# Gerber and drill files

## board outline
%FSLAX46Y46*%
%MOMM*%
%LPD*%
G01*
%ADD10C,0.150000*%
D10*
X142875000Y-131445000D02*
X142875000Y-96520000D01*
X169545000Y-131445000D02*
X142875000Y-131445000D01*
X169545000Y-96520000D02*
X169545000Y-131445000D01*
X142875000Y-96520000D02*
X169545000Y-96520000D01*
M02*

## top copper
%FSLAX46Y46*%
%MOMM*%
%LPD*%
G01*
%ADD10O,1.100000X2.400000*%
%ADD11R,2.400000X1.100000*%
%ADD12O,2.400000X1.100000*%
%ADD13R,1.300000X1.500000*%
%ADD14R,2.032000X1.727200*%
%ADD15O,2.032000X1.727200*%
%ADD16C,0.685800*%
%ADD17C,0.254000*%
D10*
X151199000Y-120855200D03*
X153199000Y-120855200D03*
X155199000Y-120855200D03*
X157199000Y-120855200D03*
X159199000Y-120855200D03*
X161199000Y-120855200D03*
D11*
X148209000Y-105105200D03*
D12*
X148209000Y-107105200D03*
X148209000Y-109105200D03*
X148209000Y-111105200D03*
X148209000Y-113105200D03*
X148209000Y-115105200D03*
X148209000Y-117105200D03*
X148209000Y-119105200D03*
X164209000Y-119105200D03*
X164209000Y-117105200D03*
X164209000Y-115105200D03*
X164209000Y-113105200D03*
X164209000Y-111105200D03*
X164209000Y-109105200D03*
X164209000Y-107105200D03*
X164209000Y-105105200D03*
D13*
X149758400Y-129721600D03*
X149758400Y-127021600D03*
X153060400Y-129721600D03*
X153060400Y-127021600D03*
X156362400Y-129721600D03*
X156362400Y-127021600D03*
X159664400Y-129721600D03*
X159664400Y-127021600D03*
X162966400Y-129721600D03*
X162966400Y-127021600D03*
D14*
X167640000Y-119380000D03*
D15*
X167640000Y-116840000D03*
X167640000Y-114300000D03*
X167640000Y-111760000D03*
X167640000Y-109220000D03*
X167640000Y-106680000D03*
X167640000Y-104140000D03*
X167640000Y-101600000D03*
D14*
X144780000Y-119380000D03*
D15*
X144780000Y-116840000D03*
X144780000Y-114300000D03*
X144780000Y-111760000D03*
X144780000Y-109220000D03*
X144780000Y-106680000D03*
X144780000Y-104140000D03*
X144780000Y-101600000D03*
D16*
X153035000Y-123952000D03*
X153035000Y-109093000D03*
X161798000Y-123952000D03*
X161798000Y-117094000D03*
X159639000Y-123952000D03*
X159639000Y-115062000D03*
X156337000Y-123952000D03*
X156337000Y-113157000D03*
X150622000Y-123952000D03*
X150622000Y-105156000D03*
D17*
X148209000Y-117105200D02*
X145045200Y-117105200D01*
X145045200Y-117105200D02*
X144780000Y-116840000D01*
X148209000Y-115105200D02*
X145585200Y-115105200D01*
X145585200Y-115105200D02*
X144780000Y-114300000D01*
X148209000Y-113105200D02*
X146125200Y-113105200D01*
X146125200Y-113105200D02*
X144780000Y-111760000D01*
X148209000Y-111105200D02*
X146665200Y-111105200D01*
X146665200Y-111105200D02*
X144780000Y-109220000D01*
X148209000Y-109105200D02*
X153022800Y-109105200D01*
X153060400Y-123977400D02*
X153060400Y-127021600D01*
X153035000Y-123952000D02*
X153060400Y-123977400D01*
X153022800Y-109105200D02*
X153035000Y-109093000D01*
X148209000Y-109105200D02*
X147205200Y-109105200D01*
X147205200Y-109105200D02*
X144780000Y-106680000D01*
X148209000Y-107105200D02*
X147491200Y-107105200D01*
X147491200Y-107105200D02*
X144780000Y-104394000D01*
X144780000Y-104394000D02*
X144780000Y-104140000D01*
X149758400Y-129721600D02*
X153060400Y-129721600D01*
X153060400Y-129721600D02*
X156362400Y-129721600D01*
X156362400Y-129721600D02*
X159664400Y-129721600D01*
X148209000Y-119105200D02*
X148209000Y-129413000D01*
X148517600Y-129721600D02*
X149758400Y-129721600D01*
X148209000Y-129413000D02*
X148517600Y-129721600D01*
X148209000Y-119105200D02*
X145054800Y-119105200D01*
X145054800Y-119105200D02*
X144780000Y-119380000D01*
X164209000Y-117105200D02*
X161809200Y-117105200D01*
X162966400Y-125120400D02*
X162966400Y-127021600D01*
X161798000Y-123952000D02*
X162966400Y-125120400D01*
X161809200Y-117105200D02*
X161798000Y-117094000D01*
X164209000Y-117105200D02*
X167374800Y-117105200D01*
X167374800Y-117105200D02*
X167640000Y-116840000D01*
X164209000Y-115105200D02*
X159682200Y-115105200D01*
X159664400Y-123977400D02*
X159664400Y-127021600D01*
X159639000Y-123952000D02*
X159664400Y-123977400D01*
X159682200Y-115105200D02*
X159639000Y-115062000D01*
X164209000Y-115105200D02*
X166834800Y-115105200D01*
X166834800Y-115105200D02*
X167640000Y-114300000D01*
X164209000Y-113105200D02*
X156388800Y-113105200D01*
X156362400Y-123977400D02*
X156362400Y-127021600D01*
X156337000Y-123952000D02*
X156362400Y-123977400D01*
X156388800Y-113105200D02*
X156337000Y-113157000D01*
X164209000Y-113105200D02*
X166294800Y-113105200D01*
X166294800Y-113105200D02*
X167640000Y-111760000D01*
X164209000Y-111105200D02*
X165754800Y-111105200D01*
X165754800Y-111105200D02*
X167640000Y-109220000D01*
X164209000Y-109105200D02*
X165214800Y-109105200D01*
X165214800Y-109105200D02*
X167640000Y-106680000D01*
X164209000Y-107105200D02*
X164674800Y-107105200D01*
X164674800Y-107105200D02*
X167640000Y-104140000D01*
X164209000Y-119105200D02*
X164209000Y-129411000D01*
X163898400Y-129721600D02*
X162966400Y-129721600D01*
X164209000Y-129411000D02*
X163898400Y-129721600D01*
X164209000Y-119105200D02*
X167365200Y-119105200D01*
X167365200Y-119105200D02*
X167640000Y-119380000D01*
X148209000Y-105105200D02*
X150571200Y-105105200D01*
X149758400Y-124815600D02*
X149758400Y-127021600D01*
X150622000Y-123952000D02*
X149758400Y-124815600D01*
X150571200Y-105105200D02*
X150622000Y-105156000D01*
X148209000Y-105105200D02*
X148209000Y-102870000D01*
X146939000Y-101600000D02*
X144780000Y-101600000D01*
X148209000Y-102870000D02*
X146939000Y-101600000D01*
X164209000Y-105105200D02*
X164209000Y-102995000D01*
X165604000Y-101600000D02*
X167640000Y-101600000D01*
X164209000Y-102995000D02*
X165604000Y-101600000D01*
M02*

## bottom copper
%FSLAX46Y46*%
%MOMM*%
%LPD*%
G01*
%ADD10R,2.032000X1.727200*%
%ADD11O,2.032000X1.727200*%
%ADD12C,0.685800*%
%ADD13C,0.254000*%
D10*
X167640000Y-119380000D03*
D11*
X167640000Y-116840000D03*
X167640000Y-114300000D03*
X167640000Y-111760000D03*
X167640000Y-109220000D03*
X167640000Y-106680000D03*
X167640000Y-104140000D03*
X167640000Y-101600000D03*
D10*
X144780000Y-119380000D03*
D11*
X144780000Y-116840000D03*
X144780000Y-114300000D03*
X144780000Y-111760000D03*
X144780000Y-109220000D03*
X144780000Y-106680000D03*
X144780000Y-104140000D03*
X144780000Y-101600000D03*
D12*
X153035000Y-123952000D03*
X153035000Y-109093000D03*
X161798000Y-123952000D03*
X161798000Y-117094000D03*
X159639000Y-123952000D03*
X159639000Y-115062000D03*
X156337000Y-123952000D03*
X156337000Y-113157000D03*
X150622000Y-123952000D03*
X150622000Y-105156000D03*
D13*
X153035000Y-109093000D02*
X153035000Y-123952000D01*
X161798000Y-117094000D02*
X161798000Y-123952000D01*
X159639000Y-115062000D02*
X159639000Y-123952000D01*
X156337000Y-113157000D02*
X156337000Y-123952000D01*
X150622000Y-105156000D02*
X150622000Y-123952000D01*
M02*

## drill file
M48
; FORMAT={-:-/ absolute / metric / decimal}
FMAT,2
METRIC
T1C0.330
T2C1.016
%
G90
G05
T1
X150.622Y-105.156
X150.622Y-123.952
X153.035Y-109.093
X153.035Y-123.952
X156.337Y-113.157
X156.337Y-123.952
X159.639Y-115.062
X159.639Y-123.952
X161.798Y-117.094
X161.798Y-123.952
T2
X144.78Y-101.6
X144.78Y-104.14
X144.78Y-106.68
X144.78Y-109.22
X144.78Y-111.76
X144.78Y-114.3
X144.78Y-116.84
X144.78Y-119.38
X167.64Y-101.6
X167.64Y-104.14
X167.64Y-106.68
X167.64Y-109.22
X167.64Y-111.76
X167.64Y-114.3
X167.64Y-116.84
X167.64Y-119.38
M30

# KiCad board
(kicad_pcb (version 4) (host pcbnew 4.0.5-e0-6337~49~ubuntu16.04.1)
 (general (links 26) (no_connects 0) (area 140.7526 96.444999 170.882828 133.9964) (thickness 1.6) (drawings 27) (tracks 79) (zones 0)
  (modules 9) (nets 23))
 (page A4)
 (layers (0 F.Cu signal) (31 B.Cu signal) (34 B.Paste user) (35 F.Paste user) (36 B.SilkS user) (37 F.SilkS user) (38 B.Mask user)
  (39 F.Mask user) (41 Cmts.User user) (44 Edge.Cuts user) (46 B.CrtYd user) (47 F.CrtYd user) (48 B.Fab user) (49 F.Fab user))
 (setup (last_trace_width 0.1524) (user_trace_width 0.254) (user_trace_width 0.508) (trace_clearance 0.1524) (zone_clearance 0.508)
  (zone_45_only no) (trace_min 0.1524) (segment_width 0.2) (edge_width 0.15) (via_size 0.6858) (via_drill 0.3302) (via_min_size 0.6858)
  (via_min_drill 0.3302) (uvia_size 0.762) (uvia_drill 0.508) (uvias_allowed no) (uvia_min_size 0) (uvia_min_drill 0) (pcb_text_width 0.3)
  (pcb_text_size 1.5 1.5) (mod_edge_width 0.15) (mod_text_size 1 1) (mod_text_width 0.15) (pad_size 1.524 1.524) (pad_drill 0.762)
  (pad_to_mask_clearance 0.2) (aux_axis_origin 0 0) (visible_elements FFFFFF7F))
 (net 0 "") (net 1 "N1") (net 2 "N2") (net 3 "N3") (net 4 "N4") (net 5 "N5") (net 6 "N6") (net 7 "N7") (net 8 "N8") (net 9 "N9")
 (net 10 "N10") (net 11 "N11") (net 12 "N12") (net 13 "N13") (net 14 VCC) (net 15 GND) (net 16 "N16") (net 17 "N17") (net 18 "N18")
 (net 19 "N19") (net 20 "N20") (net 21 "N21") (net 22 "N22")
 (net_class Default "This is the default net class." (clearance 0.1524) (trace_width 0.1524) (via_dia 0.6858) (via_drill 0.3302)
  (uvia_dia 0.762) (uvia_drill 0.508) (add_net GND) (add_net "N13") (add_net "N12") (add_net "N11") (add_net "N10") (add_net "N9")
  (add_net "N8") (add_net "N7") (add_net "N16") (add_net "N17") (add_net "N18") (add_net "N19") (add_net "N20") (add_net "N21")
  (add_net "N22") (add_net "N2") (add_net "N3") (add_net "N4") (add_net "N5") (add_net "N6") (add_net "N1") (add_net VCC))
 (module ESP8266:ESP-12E (layer F.Cu) (at 148.209 105.1052)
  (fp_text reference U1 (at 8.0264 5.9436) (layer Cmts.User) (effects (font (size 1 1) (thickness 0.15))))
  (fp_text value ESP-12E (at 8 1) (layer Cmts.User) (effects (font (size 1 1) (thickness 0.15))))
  (pad 9 smd oval (at 2.99 15.75 90) (size 2.4 1.1) (layers F.Cu F.Paste F.Mask) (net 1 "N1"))
  (pad 10 smd oval (at 4.99 15.75 90) (size 2.4 1.1) (layers F.Cu F.Paste F.Mask) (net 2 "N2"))
  (pad 11 smd oval (at 6.99 15.75 90) (size 2.4 1.1) (layers F.Cu F.Paste F.Mask) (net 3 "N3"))
  (pad 12 smd oval (at 8.99 15.75 90) (size 2.4 1.1) (layers F.Cu F.Paste F.Mask) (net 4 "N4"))
  (pad 13 smd oval (at 10.99 15.75 90) (size 2.4 1.1) (layers F.Cu F.Paste F.Mask) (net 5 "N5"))
  (pad 14 smd oval (at 12.99 15.75 90) (size 2.4 1.1) (layers F.Cu F.Paste F.Mask) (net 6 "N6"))
  (pad 1 smd rect (at 0 0) (size 2.4 1.1) (layers F.Cu F.Paste F.Mask) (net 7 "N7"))
  (pad 2 smd oval (at 0 2) (size 2.4 1.1) (layers F.Cu F.Paste F.Mask) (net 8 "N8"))
  (pad 3 smd oval (at 0 4) (size 2.4 1.1) (layers F.Cu F.Paste F.Mask) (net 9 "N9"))
  (pad 4 smd oval (at 0 6) (size 2.4 1.1) (layers F.Cu F.Paste F.Mask) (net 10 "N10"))
  (pad 5 smd oval (at 0 8) (size 2.4 1.1) (layers F.Cu F.Paste F.Mask) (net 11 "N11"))
  (pad 6 smd oval (at 0 10) (size 2.4 1.1) (layers F.Cu F.Paste F.Mask) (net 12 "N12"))
  (pad 7 smd oval (at 0 12) (size 2.4 1.1) (layers F.Cu F.Paste F.Mask) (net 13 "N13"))
  (pad 8 smd oval (at 0 14) (size 2.4 1.1) (layers F.Cu F.Paste F.Mask) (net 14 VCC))
  (pad 15 smd oval (at 16 14) (size 2.4 1.1) (layers F.Cu F.Paste F.Mask) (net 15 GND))
  (pad 16 smd oval (at 16 12) (size 2.4 1.1) (layers F.Cu F.Paste F.Mask) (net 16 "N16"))
  (pad 17 smd oval (at 16 10) (size 2.4 1.1) (layers F.Cu F.Paste F.Mask) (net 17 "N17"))
  (pad 18 smd oval (at 16 8) (size 2.4 1.1) (layers F.Cu F.Paste F.Mask) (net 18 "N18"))
  (pad 19 smd oval (at 16 6) (size 2.4 1.1) (layers F.Cu F.Paste F.Mask) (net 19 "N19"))
  (pad 20 smd oval (at 16 4) (size 2.4 1.1) (layers F.Cu F.Paste F.Mask) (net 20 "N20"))
  (pad 21 smd oval (at 16 2) (size 2.4 1.1) (layers F.Cu F.Paste F.Mask) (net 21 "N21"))
  (pad 22 smd oval (at 16 0) (size 2.4 1.1) (layers F.Cu F.Paste F.Mask) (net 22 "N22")))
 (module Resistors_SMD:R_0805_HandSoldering (layer F.Cu) (at 149.7584 128.3716 90)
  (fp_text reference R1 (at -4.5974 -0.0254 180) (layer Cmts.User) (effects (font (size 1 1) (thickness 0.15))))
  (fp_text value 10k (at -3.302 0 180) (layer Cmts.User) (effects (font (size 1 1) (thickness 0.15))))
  (pad 1 smd rect (at -1.35 0 90) (size 1.5 1.3) (layers F.Cu F.Paste F.Mask) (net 14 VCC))
  (pad 2 smd rect (at 1.35 0 90) (size 1.5 1.3) (layers F.Cu F.Paste F.Mask) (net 7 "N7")))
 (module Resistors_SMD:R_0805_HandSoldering (layer F.Cu) (at 153.0604 128.3716 90)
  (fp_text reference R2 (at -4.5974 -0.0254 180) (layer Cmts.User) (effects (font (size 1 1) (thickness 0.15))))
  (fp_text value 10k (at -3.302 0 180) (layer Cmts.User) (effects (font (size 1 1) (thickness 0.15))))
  (pad 1 smd rect (at -1.35 0 90) (size 1.5 1.3) (layers F.Cu F.Paste F.Mask) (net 14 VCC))
  (pad 2 smd rect (at 1.35 0 90) (size 1.5 1.3) (layers F.Cu F.Paste F.Mask) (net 9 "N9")))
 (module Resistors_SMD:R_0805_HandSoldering (layer F.Cu) (at 156.3624 128.3716 90)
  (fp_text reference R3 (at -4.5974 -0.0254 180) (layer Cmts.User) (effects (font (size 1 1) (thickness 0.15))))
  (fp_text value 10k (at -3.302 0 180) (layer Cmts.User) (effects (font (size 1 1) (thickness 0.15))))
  (pad 1 smd rect (at -1.35 0 90) (size 1.5 1.3) (layers F.Cu F.Paste F.Mask) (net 14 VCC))
  (pad 2 smd rect (at 1.35 0 90) (size 1.5 1.3) (layers F.Cu F.Paste F.Mask) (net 18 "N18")))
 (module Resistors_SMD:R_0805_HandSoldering (layer F.Cu) (at 159.6644 128.3716 90)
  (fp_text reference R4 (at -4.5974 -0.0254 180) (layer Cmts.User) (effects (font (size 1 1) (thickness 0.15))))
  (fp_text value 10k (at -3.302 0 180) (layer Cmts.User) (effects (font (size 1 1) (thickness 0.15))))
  (pad 1 smd rect (at -1.35 0 90) (size 1.5 1.3) (layers F.Cu F.Paste F.Mask) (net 14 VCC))
  (pad 2 smd rect (at 1.35 0 90) (size 1.5 1.3) (layers F.Cu F.Paste F.Mask) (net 17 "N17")))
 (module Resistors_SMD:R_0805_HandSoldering (layer F.Cu) (at 162.9664 128.3716 90)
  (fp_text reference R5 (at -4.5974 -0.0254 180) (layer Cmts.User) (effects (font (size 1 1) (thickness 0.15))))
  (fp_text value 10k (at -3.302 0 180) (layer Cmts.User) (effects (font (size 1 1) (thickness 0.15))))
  (pad 1 smd rect (at -1.35 0 90) (size 1.5 1.3) (layers F.Cu F.Paste F.Mask) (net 15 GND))
  (pad 2 smd rect (at 1.35 0 90) (size 1.5 1.3) (layers F.Cu F.Paste F.Mask) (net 16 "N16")))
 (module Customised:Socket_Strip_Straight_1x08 (layer F.Cu) (at 167.64 119.38 90)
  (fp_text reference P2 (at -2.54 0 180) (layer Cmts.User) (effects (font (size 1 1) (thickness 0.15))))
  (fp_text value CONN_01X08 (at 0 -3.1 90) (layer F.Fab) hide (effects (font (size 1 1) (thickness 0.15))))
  (pad 1 thru_hole rect (at 0 0 90) (size 1.7272 2.032) (drill 1.016) (layers *.Cu *.Mask) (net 15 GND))
  (pad 2 thru_hole oval (at 2.54 0 90) (size 1.7272 2.032) (drill 1.016) (layers *.Cu *.Mask) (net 16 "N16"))
  (pad 3 thru_hole oval (at 5.08 0 90) (size 1.7272 2.032) (drill 1.016) (layers *.Cu *.Mask) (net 17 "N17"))
  (pad 4 thru_hole oval (at 7.62 0 90) (size 1.7272 2.032) (drill 1.016) (layers *.Cu *.Mask) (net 18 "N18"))
  (pad 5 thru_hole oval (at 10.16 0 90) (size 1.7272 2.032) (drill 1.016) (layers *.Cu *.Mask) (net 19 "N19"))
  (pad 6 thru_hole oval (at 12.7 0 90) (size 1.7272 2.032) (drill 1.016) (layers *.Cu *.Mask) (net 20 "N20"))
  (pad 7 thru_hole oval (at 15.24 0 90) (size 1.7272 2.032) (drill 1.016) (layers *.Cu *.Mask) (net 21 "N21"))
  (pad 8 thru_hole oval (at 17.78 0 90) (size 1.7272 2.032) (drill 1.016) (layers *.Cu *.Mask) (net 22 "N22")))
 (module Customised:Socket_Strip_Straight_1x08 (layer F.Cu) (at 144.78 119.38 90)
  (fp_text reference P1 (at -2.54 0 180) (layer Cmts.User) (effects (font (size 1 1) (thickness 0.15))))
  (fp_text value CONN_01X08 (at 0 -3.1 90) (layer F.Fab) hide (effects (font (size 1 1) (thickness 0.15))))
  (pad 1 thru_hole rect (at 0 0 90) (size 1.7272 2.032) (drill 1.016) (layers *.Cu *.Mask) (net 14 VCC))
  (pad 2 thru_hole oval (at 2.54 0 90) (size 1.7272 2.032) (drill 1.016) (layers *.Cu *.Mask) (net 13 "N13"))
  (pad 3 thru_hole oval (at 5.08 0 90) (size 1.7272 2.032) (drill 1.016) (layers *.Cu *.Mask) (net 12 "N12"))
  (pad 4 thru_hole oval (at 7.62 0 90) (size 1.7272 2.032) (drill 1.016) (layers *.Cu *.Mask) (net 11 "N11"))
  (pad 5 thru_hole oval (at 10.16 0 90) (size 1.7272 2.032) (drill 1.016) (layers *.Cu *.Mask) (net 10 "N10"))
  (pad 6 thru_hole oval (at 12.7 0 90) (size 1.7272 2.032) (drill 1.016) (layers *.Cu *.Mask) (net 9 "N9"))
  (pad 7 thru_hole oval (at 15.24 0 90) (size 1.7272 2.032) (drill 1.016) (layers *.Cu *.Mask) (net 8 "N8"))
  (pad 8 thru_hole oval (at 17.78 0 90) (size 1.7272 2.032) (drill 1.016) (layers *.Cu *.Mask) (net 7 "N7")))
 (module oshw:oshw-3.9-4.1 (layer F.Cu) (at 167.005 128.27)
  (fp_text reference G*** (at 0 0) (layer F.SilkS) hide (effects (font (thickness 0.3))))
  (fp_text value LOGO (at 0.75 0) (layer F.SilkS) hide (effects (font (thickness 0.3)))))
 (gr_line (start 142.875 131.445) (end 142.875 96.52) (angle 90) (layer Edge.Cuts) (width 0.15))
 (gr_line (start 169.545 131.445) (end 142.875 131.445) (angle 90) (layer Edge.Cuts) (width 0.15))
 (gr_line (start 169.545 96.52) (end 169.545 131.445) (angle 90) (layer Edge.Cuts) (width 0.15))
 (gr_line (start 142.875 96.52) (end 169.545 96.52) (angle 90) (layer Edge.Cuts) (width 0.15))
 (segment (start 148.209 117.1052) (end 145.0452 117.1052) (width 0.254) (layer F.Cu) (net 13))
 (segment (start 145.0452 117.1052) (end 144.78 116.84) (width 0.254) (layer F.Cu) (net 13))
 (segment (start 148.209 115.1052) (end 145.5852 115.1052) (width 0.254) (layer F.Cu) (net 12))
 (segment (start 145.5852 115.1052) (end 144.78 114.3) (width 0.254) (layer F.Cu) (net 12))
 (segment (start 148.209 113.1052) (end 146.1252 113.1052) (width 0.254) (layer F.Cu) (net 11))
 (segment (start 146.1252 113.1052) (end 144.78 111.76) (width 0.254) (layer F.Cu) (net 11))
 (segment (start 148.209 111.1052) (end 146.6652 111.1052) (width 0.254) (layer F.Cu) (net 10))
 (segment (start 146.6652 111.1052) (end 144.78 109.22) (width 0.254) (layer F.Cu) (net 10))
 (segment (start 148.209 109.1052) (end 153.0228 109.1052) (width 0.254) (layer F.Cu) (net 9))
 (segment (start 153.0604 123.9774) (end 153.0604 127.0216) (width 0.254) (layer F.Cu) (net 9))
 (segment (start 153.035 123.952) (end 153.0604 123.9774) (width 0.254) (layer F.Cu) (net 9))
 (segment (start 153.035 109.093) (end 153.035 123.952) (width 0.254) (layer B.Cu) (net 9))
 (segment (start 153.0228 109.1052) (end 153.035 109.093) (width 0.254) (layer F.Cu) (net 9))
 (segment (start 148.209 109.1052) (end 147.2052 109.1052) (width 0.254) (layer F.Cu) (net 9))
 (segment (start 147.2052 109.1052) (end 144.78 106.68) (width 0.254) (layer F.Cu) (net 9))
 (segment (start 148.209 107.1052) (end 147.4912 107.1052) (width 0.254) (layer F.Cu) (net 8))
 (segment (start 147.4912 107.1052) (end 144.78 104.394) (width 0.254) (layer F.Cu) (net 8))
 (segment (start 144.78 104.394) (end 144.78 104.14) (width 0.254) (layer F.Cu) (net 8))
 (segment (start 149.7584 129.7216) (end 153.0604 129.7216) (width 0.254) (layer F.Cu) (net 14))
 (segment (start 153.0604 129.7216) (end 156.3624 129.7216) (width 0.254) (layer F.Cu) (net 14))
 (segment (start 156.3624 129.7216) (end 159.6644 129.7216) (width 0.254) (layer F.Cu) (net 14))
 (segment (start 148.209 119.1052) (end 148.209 129.413) (width 0.254) (layer F.Cu) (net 14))
 (segment (start 148.5176 129.7216) (end 149.7584 129.7216) (width 0.254) (layer F.Cu) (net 14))
 (segment (start 148.209 129.413) (end 148.5176 129.7216) (width 0.254) (layer F.Cu) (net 14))
 (segment (start 148.209 119.1052) (end 145.0548 119.1052) (width 0.254) (layer F.Cu) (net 14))
 (segment (start 145.0548 119.1052) (end 144.78 119.38) (width 0.254) (layer F.Cu) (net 14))
 (segment (start 164.209 117.1052) (end 161.8092 117.1052) (width 0.254) (layer F.Cu) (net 16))
 (segment (start 162.9664 125.1204) (end 162.9664 127.0216) (width 0.254) (layer F.Cu) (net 16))
 (segment (start 161.798 123.952) (end 162.9664 125.1204) (width 0.254) (layer F.Cu) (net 16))
 (segment (start 161.798 117.094) (end 161.798 123.952) (width 0.254) (layer B.Cu) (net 16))
 (segment (start 161.8092 117.1052) (end 161.798 117.094) (width 0.254) (layer F.Cu) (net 16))
 (segment (start 164.209 117.1052) (end 167.3748 117.1052) (width 0.254) (layer F.Cu) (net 16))
 (segment (start 167.3748 117.1052) (end 167.64 116.84) (width 0.254) (layer F.Cu) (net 16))
 (segment (start 164.209 115.1052) (end 159.6822 115.1052) (width 0.254) (layer F.Cu) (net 17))
 (segment (start 159.6644 123.9774) (end 159.6644 127.0216) (width 0.254) (layer F.Cu) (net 17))
 (segment (start 159.639 123.952) (end 159.6644 123.9774) (width 0.254) (layer F.Cu) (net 17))
 (segment (start 159.639 115.062) (end 159.639 123.952) (width 0.254) (layer B.Cu) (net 17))
 (segment (start 159.6822 115.1052) (end 159.639 115.062) (width 0.254) (layer F.Cu) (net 17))
 (segment (start 164.209 115.1052) (end 166.8348 115.1052) (width 0.254) (layer F.Cu) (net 17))
 (segment (start 166.8348 115.1052) (end 167.64 114.3) (width 0.254) (layer F.Cu) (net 17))
 (segment (start 164.209 113.1052) (end 156.3888 113.1052) (width 0.254) (layer F.Cu) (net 18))
 (segment (start 156.3624 123.9774) (end 156.3624 127.0216) (width 0.254) (layer F.Cu) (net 18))
 (segment (start 156.337 123.952) (end 156.3624 123.9774) (width 0.254) (layer F.Cu) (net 18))
 (segment (start 156.337 113.157) (end 156.337 123.952) (width 0.254) (layer B.Cu) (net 18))
 (segment (start 156.3888 113.1052) (end 156.337 113.157) (width 0.254) (layer F.Cu) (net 18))
 (segment (start 164.209 113.1052) (end 166.2948 113.1052) (width 0.254) (layer F.Cu) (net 18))
 (segment (start 166.2948 113.1052) (end 167.64 111.76) (width 0.254) (layer F.Cu) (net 18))
 (segment (start 164.209 111.1052) (end 165.7548 111.1052) (width 0.254) (layer F.Cu) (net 19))
 (segment (start 165.7548 111.1052) (end 167.64 109.22) (width 0.254) (layer F.Cu) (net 19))
 (segment (start 164.209 109.1052) (end 165.2148 109.1052) (width 0.254) (layer F.Cu) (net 20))
 (segment (start 165.2148 109.1052) (end 167.64 106.68) (width 0.254) (layer F.Cu) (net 20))
 (segment (start 164.209 107.1052) (end 164.6748 107.1052) (width 0.254) (layer F.Cu) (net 21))
 (segment (start 164.6748 107.1052) (end 167.64 104.14) (width 0.254) (layer F.Cu) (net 21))
 (segment (start 164.209 119.1052) (end 164.209 129.411) (width 0.254) (layer F.Cu) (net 15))
 (segment (start 163.8984 129.7216) (end 162.9664 129.7216) (width 0.254) (layer F.Cu) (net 15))
 (segment (start 164.209 129.411) (end 163.8984 129.7216) (width 0.254) (layer F.Cu) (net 15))
 (segment (start 164.209 119.1052) (end 167.3652 119.1052) (width 0.254) (layer F.Cu) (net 15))
 (segment (start 167.3652 119.1052) (end 167.64 119.38) (width 0.254) (layer F.Cu) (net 15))
 (segment (start 148.209 105.1052) (end 150.5712 105.1052) (width 0.254) (layer F.Cu) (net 7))
 (segment (start 149.7584 124.8156) (end 149.7584 127.0216) (width 0.254) (layer F.Cu) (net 7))
 (segment (start 150.622 123.952) (end 149.7584 124.8156) (width 0.254) (layer F.Cu) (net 7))
 (segment (start 150.622 105.156) (end 150.622 123.952) (width 0.254) (layer B.Cu) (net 7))
 (segment (start 150.5712 105.1052) (end 150.622 105.156) (width 0.254) (layer F.Cu) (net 7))
 (segment (start 148.209 105.1052) (end 148.209 102.87) (width 0.254) (layer F.Cu) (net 7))
 (segment (start 146.939 101.6) (end 144.78 101.6) (width 0.254) (layer F.Cu) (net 7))
 (segment (start 148.209 102.87) (end 146.939 101.6) (width 0.254) (layer F.Cu) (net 7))
 (segment (start 164.209 105.1052) (end 164.209 102.995) (width 0.254) (layer F.Cu) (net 22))
 (segment (start 165.604 101.6) (end 167.64 101.6) (width 0.254) (layer F.Cu) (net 22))
 (segment (start 164.209 102.995) (end 165.604 101.6) (width 0.254) (layer F.Cu) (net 22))
 (via (at 153.035 123.952) (size 0.6858) (drill 0.3302) (layers F.Cu B.Cu) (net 9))
 (via (at 153.035 109.093) (size 0.6858) (drill 0.3302) (layers F.Cu B.Cu) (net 9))
 (via (at 161.798 123.952) (size 0.6858) (drill 0.3302) (layers F.Cu B.Cu) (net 16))
 (via (at 161.798 117.094) (size 0.6858) (drill 0.3302) (layers F.Cu B.Cu) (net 16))
 (via (at 159.639 123.952) (size 0.6858) (drill 0.3302) (layers F.Cu B.Cu) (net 17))
 (via (at 159.639 115.062) (size 0.6858) (drill 0.3302) (layers F.Cu B.Cu) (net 17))
 (via (at 156.337 123.952) (size 0.6858) (drill 0.3302) (layers F.Cu B.Cu) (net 18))
 (via (at 156.337 113.157) (size 0.6858) (drill 0.3302) (layers F.Cu B.Cu) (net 18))
 (via (at 150.622 123.952) (size 0.6858) (drill 0.3302) (layers F.Cu B.Cu) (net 7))
 (via (at 150.622 105.156) (size 0.6858) (drill 0.3302) (layers F.Cu B.Cu) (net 7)))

